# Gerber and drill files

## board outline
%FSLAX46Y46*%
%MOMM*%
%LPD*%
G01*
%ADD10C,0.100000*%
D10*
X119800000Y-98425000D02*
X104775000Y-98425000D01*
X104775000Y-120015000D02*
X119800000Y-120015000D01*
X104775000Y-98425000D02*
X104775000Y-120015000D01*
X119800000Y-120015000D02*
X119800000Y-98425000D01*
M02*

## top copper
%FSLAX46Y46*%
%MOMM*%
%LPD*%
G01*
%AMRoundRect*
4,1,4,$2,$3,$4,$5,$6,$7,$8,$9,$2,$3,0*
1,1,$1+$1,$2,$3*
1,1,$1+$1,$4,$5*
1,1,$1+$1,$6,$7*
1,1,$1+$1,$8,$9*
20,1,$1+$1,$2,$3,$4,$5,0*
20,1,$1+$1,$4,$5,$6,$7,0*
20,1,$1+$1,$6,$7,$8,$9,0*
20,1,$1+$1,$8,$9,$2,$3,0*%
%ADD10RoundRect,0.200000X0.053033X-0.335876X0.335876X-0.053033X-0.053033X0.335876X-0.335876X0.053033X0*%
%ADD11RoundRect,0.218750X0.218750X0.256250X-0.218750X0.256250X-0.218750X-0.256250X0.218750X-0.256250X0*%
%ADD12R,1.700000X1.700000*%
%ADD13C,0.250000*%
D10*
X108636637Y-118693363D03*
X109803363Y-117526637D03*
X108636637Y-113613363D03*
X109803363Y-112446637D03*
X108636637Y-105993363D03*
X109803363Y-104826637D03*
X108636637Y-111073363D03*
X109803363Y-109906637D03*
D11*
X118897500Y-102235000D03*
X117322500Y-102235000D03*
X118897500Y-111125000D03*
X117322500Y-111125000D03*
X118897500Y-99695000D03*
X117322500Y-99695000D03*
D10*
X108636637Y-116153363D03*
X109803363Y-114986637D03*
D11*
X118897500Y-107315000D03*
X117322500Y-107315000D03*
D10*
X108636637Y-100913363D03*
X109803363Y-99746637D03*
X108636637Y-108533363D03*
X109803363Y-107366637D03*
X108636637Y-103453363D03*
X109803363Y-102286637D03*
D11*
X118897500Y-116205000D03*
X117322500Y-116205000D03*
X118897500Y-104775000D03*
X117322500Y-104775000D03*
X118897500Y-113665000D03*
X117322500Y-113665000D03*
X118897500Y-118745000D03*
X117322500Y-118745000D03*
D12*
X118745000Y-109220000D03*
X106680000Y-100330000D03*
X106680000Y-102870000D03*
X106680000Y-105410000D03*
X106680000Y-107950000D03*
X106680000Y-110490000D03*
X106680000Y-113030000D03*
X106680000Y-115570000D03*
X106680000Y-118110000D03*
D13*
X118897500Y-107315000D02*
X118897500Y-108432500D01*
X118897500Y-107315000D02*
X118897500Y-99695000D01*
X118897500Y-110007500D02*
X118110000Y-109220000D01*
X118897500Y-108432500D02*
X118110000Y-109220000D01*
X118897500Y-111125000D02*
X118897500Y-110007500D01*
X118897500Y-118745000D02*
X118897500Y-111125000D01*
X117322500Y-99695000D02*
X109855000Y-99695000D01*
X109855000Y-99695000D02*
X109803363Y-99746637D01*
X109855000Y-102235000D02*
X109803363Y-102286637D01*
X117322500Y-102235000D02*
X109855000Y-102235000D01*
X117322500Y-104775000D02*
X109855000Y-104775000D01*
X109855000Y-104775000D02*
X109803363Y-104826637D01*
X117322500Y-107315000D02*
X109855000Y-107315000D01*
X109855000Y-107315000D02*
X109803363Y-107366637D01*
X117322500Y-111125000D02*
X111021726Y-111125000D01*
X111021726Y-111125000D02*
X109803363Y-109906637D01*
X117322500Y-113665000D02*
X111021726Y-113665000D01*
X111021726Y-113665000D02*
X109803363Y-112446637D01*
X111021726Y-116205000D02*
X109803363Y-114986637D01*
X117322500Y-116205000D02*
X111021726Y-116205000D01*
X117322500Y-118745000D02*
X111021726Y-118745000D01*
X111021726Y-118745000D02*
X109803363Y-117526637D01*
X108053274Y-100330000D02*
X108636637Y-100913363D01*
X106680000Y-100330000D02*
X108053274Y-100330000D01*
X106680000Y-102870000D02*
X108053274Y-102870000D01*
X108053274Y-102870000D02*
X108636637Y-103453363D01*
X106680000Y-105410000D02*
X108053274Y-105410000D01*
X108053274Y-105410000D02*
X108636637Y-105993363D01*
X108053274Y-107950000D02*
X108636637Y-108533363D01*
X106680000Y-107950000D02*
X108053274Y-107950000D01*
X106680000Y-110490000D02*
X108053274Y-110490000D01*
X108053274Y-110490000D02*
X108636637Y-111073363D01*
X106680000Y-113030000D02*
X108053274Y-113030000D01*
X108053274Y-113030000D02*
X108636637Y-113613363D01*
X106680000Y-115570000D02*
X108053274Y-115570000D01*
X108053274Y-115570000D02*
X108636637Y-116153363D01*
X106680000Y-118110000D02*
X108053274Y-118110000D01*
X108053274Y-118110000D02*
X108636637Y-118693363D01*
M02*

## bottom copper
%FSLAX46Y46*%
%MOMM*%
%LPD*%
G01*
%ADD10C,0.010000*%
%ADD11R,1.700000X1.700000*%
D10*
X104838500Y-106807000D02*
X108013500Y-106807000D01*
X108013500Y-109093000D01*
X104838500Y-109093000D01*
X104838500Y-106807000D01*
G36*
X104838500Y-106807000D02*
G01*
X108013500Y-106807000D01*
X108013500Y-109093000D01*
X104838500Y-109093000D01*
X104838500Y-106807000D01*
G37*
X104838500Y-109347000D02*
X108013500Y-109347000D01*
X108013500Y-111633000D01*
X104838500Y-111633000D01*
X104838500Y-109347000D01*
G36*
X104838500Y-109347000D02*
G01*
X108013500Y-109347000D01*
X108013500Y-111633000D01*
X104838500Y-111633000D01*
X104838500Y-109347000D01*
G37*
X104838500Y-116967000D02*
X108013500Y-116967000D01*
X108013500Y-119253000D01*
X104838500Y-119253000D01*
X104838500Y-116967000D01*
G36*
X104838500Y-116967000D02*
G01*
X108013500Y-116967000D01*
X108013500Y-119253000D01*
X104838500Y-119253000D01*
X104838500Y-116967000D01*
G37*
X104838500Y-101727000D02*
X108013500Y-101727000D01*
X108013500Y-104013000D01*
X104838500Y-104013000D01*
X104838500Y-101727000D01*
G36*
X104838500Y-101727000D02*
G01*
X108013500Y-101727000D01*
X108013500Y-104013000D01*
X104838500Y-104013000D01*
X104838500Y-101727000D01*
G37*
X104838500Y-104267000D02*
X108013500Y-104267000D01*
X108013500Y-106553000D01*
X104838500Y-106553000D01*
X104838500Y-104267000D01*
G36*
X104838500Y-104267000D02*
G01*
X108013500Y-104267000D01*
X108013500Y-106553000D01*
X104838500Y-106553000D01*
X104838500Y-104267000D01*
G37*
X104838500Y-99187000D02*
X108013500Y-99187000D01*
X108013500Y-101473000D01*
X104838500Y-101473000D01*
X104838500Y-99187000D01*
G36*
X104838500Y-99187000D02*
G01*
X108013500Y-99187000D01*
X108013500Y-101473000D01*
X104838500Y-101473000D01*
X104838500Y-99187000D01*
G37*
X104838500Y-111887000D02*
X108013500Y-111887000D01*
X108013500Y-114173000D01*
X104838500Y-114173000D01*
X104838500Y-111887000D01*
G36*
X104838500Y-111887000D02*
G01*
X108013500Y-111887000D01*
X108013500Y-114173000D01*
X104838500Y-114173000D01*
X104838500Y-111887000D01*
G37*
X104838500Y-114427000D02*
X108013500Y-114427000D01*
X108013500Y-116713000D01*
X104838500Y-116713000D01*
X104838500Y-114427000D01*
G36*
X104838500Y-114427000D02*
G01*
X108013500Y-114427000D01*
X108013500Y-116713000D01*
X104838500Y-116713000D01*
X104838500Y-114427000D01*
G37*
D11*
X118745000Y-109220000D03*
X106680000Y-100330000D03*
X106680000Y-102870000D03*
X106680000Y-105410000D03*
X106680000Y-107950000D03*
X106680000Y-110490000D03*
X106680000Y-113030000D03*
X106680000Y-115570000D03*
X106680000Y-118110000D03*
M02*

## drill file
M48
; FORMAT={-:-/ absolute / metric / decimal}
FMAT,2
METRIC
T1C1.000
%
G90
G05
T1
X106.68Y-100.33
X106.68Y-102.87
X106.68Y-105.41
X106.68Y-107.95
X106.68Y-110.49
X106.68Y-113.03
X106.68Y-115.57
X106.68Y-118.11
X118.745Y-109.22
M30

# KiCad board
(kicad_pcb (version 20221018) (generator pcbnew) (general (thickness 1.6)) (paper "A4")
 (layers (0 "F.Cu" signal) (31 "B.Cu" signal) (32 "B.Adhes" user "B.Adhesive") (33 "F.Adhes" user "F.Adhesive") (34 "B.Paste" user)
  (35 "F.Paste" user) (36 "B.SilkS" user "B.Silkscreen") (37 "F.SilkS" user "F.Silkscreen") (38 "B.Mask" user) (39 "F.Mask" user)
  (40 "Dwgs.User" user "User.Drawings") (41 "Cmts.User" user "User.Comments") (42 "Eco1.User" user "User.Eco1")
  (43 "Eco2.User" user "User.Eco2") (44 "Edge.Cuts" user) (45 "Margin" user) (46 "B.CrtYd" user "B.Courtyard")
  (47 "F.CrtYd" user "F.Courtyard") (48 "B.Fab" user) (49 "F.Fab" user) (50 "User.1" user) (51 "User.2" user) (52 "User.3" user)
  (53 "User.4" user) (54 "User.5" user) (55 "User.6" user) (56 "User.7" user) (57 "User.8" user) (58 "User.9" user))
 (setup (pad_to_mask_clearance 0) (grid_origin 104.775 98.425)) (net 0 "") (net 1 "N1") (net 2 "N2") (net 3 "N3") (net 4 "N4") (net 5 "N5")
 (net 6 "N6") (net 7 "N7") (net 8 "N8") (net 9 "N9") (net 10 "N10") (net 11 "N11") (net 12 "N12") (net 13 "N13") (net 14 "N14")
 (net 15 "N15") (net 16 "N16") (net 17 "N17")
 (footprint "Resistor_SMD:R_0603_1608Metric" (layer "F.Cu") (at 109.22 118.11 45)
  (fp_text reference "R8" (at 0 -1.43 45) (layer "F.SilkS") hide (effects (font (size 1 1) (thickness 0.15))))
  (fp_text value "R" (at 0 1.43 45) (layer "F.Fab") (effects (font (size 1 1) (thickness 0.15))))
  (pad "1" smd roundrect (at -0.825 0 45) (size 0.8 0.95) (layers "F.Cu" "F.Paste" "F.Mask") (roundrect_rratio 0.25) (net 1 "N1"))
  (pad "2" smd roundrect (at 0.825 0 45) (size 0.8 0.95) (layers "F.Cu" "F.Paste" "F.Mask") (roundrect_rratio 0.25) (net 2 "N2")))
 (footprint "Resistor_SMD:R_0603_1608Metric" (layer "F.Cu") (at 109.22 113.03 45)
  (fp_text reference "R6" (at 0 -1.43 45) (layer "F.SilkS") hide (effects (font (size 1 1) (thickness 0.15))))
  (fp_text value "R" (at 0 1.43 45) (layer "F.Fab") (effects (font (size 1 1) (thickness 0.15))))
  (pad "1" smd roundrect (at -0.825 0 45) (size 0.8 0.95) (layers "F.Cu" "F.Paste" "F.Mask") (roundrect_rratio 0.25) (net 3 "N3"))
  (pad "2" smd roundrect (at 0.825 0 45) (size 0.8 0.95) (layers "F.Cu" "F.Paste" "F.Mask") (roundrect_rratio 0.25) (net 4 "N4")))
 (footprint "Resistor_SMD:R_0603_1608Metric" (layer "F.Cu") (at 109.22 105.41 45)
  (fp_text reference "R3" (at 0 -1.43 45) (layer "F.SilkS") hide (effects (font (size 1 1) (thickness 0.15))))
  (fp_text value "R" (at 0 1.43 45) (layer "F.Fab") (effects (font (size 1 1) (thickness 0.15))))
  (pad "1" smd roundrect (at -0.825 0 45) (size 0.8 0.95) (layers "F.Cu" "F.Paste" "F.Mask") (roundrect_rratio 0.25) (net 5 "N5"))
  (pad "2" smd roundrect (at 0.825 0 45) (size 0.8 0.95) (layers "F.Cu" "F.Paste" "F.Mask") (roundrect_rratio 0.25) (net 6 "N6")))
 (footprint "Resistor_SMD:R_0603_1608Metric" (layer "F.Cu") (at 109.22 110.49 45)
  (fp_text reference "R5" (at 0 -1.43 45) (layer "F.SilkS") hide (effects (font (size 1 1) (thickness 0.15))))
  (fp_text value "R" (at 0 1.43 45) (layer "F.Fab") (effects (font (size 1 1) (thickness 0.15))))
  (pad "1" smd roundrect (at -0.825 0 45) (size 0.8 0.95) (layers "F.Cu" "F.Paste" "F.Mask") (roundrect_rratio 0.25) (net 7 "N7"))
  (pad "2" smd roundrect (at 0.825 0 45) (size 0.8 0.95) (layers "F.Cu" "F.Paste" "F.Mask") (roundrect_rratio 0.25) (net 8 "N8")))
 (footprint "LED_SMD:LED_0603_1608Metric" (layer "F.Cu") (at 118.11 102.235 180)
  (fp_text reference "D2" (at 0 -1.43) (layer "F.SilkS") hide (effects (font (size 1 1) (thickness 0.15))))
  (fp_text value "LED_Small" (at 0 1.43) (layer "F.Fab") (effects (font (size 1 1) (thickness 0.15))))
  (pad "1" smd roundrect (at -0.7875 0 180) (size 0.875 0.95) (layers "F.Cu" "F.Paste" "F.Mask") (roundrect_rratio 0.25) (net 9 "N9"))
  (pad "2" smd roundrect (at 0.7875 0 180) (size 0.875 0.95) (layers "F.Cu" "F.Paste" "F.Mask") (roundrect_rratio 0.25) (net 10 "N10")))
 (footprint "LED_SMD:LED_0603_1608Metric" (layer "F.Cu") (at 118.11 111.125 180)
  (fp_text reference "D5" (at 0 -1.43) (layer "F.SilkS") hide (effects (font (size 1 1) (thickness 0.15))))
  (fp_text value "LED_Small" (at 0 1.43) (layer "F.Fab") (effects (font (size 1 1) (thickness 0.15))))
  (pad "1" smd roundrect (at -0.7875 0 180) (size 0.875 0.95) (layers "F.Cu" "F.Paste" "F.Mask") (roundrect_rratio 0.25) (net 9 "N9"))
  (pad "2" smd roundrect (at 0.7875 0 180) (size 0.875 0.95) (layers "F.Cu" "F.Paste" "F.Mask") (roundrect_rratio 0.25) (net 8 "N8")))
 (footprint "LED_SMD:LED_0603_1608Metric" (layer "F.Cu") (at 118.11 99.695 180)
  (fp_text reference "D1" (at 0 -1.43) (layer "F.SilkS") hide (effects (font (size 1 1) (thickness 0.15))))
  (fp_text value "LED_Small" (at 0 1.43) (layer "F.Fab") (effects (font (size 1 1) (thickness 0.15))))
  (pad "1" smd roundrect (at -0.7875 0 180) (size 0.875 0.95) (layers "F.Cu" "F.Paste" "F.Mask") (roundrect_rratio 0.25) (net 9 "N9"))
  (pad "2" smd roundrect (at 0.7875 0 180) (size 0.875 0.95) (layers "F.Cu" "F.Paste" "F.Mask") (roundrect_rratio 0.25) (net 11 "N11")))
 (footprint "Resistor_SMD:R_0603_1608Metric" (layer "F.Cu") (at 109.22 115.57 45)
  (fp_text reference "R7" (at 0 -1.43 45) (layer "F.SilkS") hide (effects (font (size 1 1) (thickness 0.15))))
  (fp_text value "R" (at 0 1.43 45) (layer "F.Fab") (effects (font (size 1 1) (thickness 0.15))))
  (pad "1" smd roundrect (at -0.825 0 45) (size 0.8 0.95) (layers "F.Cu" "F.Paste" "F.Mask") (roundrect_rratio 0.25) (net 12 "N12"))
  (pad "2" smd roundrect (at 0.825 0 45) (size 0.8 0.95) (layers "F.Cu" "F.Paste" "F.Mask") (roundrect_rratio 0.25) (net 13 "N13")))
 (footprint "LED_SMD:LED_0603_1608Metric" (layer "F.Cu") (at 118.11 107.315 180)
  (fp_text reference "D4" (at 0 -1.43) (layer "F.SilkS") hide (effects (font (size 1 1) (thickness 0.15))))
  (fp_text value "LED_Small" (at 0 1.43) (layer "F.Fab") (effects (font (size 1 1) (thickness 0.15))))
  (pad "1" smd roundrect (at -0.7875 0 180) (size 0.875 0.95) (layers "F.Cu" "F.Paste" "F.Mask") (roundrect_rratio 0.25) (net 9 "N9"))
  (pad "2" smd roundrect (at 0.7875 0 180) (size 0.875 0.95) (layers "F.Cu" "F.Paste" "F.Mask") (roundrect_rratio 0.25) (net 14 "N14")))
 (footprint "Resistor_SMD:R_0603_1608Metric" (layer "F.Cu") (at 109.22 100.33 45)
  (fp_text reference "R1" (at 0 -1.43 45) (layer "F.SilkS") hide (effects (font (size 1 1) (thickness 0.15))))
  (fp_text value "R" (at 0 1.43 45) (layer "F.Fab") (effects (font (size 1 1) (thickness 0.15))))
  (pad "1" smd roundrect (at -0.825 0 45) (size 0.8 0.95) (layers "F.Cu" "F.Paste" "F.Mask") (roundrect_rratio 0.25) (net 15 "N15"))
  (pad "2" smd roundrect (at 0.825 0 45) (size 0.8 0.95) (layers "F.Cu" "F.Paste" "F.Mask") (roundrect_rratio 0.25) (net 11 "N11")))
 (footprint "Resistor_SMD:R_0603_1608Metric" (layer "F.Cu") (at 109.22 107.95 45)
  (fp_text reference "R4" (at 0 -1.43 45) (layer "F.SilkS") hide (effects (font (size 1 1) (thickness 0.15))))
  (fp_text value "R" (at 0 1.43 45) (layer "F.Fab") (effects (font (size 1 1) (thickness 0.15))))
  (pad "1" smd roundrect (at -0.825 0 45) (size 0.8 0.95) (layers "F.Cu" "F.Paste" "F.Mask") (roundrect_rratio 0.25) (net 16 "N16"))
  (pad "2" smd roundrect (at 0.825 0 45) (size 0.8 0.95) (layers "F.Cu" "F.Paste" "F.Mask") (roundrect_rratio 0.25) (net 14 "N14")))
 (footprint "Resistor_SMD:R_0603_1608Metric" (layer "F.Cu") (at 109.22 102.87 45)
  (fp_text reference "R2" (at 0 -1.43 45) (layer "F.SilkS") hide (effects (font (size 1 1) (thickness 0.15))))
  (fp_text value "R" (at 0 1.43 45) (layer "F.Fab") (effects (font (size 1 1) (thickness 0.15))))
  (pad "1" smd roundrect (at -0.825 0 45) (size 0.8 0.95) (layers "F.Cu" "F.Paste" "F.Mask") (roundrect_rratio 0.25) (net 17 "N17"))
  (pad "2" smd roundrect (at 0.825 0 45) (size 0.8 0.95) (layers "F.Cu" "F.Paste" "F.Mask") (roundrect_rratio 0.25) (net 10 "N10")))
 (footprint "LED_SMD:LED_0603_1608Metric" (layer "F.Cu") (at 118.11 116.205 180)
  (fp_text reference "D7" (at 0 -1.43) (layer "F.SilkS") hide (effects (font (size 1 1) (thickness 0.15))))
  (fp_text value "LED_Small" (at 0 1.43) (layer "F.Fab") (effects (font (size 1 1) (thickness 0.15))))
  (pad "1" smd roundrect (at -0.7875 0 180) (size 0.875 0.95) (layers "F.Cu" "F.Paste" "F.Mask") (roundrect_rratio 0.25) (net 9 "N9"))
  (pad "2" smd roundrect (at 0.7875 0 180) (size 0.875 0.95) (layers "F.Cu" "F.Paste" "F.Mask") (roundrect_rratio 0.25) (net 13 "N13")))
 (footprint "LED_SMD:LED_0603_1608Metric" (layer "F.Cu") (at 118.11 104.775 180)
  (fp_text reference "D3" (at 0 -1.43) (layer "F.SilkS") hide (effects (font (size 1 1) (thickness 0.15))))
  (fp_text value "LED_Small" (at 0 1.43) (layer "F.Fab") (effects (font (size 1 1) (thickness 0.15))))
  (pad "1" smd roundrect (at -0.7875 0 180) (size 0.875 0.95) (layers "F.Cu" "F.Paste" "F.Mask") (roundrect_rratio 0.25) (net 9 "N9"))
  (pad "2" smd roundrect (at 0.7875 0 180) (size 0.875 0.95) (layers "F.Cu" "F.Paste" "F.Mask") (roundrect_rratio 0.25) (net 6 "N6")))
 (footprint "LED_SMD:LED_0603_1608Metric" (layer "F.Cu") (at 118.11 113.665 180)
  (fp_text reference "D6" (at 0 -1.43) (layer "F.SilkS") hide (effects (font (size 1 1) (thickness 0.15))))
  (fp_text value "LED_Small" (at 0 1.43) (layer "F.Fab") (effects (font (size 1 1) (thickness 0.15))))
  (pad "1" smd roundrect (at -0.7875 0 180) (size 0.875 0.95) (layers "F.Cu" "F.Paste" "F.Mask") (roundrect_rratio 0.25) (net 9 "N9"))
  (pad "2" smd roundrect (at 0.7875 0 180) (size 0.875 0.95) (layers "F.Cu" "F.Paste" "F.Mask") (roundrect_rratio 0.25) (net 4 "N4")))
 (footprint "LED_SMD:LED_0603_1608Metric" (layer "F.Cu") (at 118.11 118.745 180)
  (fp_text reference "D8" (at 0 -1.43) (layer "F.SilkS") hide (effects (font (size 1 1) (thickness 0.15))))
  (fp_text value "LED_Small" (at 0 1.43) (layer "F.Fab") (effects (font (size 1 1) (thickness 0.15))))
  (pad "1" smd roundrect (at -0.7875 0 180) (size 0.875 0.95) (layers "F.Cu" "F.Paste" "F.Mask") (roundrect_rratio 0.25) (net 9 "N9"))
  (pad "2" smd roundrect (at 0.7875 0 180) (size 0.875 0.95) (layers "F.Cu" "F.Paste" "F.Mask") (roundrect_rratio 0.25) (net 2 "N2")))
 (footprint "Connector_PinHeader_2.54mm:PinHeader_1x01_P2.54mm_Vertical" (layer "F.Cu") (at 118.745 109.22)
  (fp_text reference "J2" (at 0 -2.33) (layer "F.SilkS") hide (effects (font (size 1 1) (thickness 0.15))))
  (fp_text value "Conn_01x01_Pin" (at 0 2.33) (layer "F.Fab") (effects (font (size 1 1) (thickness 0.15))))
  (pad "1" thru_hole rect (at 0 0) (size 1.7 1.7) (drill 1) (layers "*.Cu" "*.Mask") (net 9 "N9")))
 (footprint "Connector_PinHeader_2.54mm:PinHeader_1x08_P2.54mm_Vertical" (layer "B.Cu") (at 106.68 100.33 180)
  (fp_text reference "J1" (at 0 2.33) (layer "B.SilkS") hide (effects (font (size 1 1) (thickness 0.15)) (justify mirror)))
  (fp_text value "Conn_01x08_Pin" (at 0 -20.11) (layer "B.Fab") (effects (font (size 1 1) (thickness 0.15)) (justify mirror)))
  (pad "1" thru_hole rect (at 0 0 180) (size 1.7 1.7) (drill 1) (layers "*.Cu" "*.Mask") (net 15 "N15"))
  (pad "2" thru_hole rect (at 0 -2.54 180) (size 1.7 1.7) (drill 1) (layers "*.Cu" "*.Mask") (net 17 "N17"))
  (pad "3" thru_hole rect (at 0 -5.08 180) (size 1.7 1.7) (drill 1) (layers "*.Cu" "*.Mask") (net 5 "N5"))
  (pad "4" thru_hole rect (at 0 -7.62 180) (size 1.7 1.7) (drill 1) (layers "*.Cu" "*.Mask") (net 16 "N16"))
  (pad "5" thru_hole rect (at 0 -10.16 180) (size 1.7 1.7) (drill 1) (layers "*.Cu" "*.Mask") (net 7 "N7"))
  (pad "6" thru_hole rect (at 0 -12.7 180) (size 1.7 1.7) (drill 1) (layers "*.Cu" "*.Mask") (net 3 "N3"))
  (pad "7" thru_hole rect (at 0 -15.24 180) (size 1.7 1.7) (drill 1) (layers "*.Cu" "*.Mask") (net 12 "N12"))
  (pad "8" thru_hole rect (at 0 -17.78 180) (size 1.7 1.7) (drill 1) (layers "*.Cu" "*.Mask") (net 1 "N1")))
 (gr_rect (start 104.8385 106.807) (end 108.0135 109.093) (stroke (width 0.01) (type solid)) (fill solid) (layer "B.Cu"))
 (gr_rect (start 104.8385 109.347) (end 108.0135 111.633) (stroke (width 0.01) (type solid)) (fill solid) (layer "B.Cu"))
 (gr_rect (start 104.8385 116.967) (end 108.0135 119.253) (stroke (width 0.01) (type solid)) (fill solid) (layer "B.Cu"))
 (gr_rect (start 104.8385 101.727) (end 108.0135 104.013) (stroke (width 0.01) (type solid)) (fill solid) (layer "B.Cu"))
 (gr_rect (start 104.8385 104.267) (end 108.0135 106.553) (stroke (width 0.01) (type solid)) (fill solid) (layer "B.Cu"))
 (gr_rect (start 104.8385 99.187) (end 108.0135 101.473) (stroke (width 0.01) (type solid)) (fill solid) (layer "B.Cu"))
 (gr_rect (start 104.8385 111.887) (end 108.0135 114.173) (stroke (width 0.01) (type solid)) (fill solid) (layer "B.Cu"))
 (gr_rect (start 104.8385 114.427) (end 108.0135 116.713) (stroke (width 0.01) (type solid)) (fill solid) (layer "B.Cu"))
 (gr_line (start 119.8 98.425) (end 104.775 98.425) (stroke (width 0.1) (type default)) (layer "Edge.Cuts"))
 (gr_line (start 104.775 120.015) (end 119.8 120.015) (stroke (width 0.1) (type default)) (layer "Edge.Cuts"))
 (gr_line (start 104.775 98.425) (end 104.775 120.015) (stroke (width 0.1) (type default)) (layer "Edge.Cuts"))
 (gr_line (start 119.8 120.015) (end 119.8 98.425) (stroke (width 0.1) (type default)) (layer "Edge.Cuts"))
 (segment (start 118.8975 107.315) (end 118.8975 108.4325) (width 0.25) (layer "F.Cu") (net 9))
 (segment (start 118.8975 107.315) (end 118.8975 99.695) (width 0.25) (layer "F.Cu") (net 9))
 (segment (start 118.8975 110.0075) (end 118.11 109.22) (width 0.25) (layer "F.Cu") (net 9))
 (segment (start 118.8975 108.4325) (end 118.11 109.22) (width 0.25) (layer "F.Cu") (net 9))
 (segment (start 118.8975 111.125) (end 118.8975 110.0075) (width 0.25) (layer "F.Cu") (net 9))
 (segment (start 118.8975 118.745) (end 118.8975 111.125) (width 0.25) (layer "F.Cu") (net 9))
 (segment (start 117.3225 99.695) (end 109.855 99.695) (width 0.25) (layer "F.Cu") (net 11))
 (segment (start 109.855 99.695) (end 109.803363 99.746637) (width 0.25) (layer "F.Cu") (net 11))
 (segment (start 109.855 102.235) (end 109.803363 102.286637) (width 0.25) (layer "F.Cu") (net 10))
 (segment (start 117.3225 102.235) (end 109.855 102.235) (width 0.25) (layer "F.Cu") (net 10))
 (segment (start 117.3225 104.775) (end 109.855 104.775) (width 0.25) (layer "F.Cu") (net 6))
 (segment (start 109.855 104.775) (end 109.803363 104.826637) (width 0.25) (layer "F.Cu") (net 6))
 (segment (start 117.3225 107.315) (end 109.855 107.315) (width 0.25) (layer "F.Cu") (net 14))
 (segment (start 109.855 107.315) (end 109.803363 107.366637) (width 0.25) (layer "F.Cu") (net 14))
 (segment (start 117.3225 111.125) (end 111.021726 111.125) (width 0.25) (layer "F.Cu") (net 8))
 (segment (start 111.021726 111.125) (end 109.803363 109.906637) (width 0.25) (layer "F.Cu") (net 8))
 (segment (start 117.3225 113.665) (end 111.021726 113.665) (width 0.25) (layer "F.Cu") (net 4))
 (segment (start 111.021726 113.665) (end 109.803363 112.446637) (width 0.25) (layer "F.Cu") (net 4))
 (segment (start 111.021726 116.205) (end 109.803363 114.986637) (width 0.25) (layer "F.Cu") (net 13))
 (segment (start 117.3225 116.205) (end 111.021726 116.205) (width 0.25) (layer "F.Cu") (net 13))
 (segment (start 117.3225 118.745) (end 111.021726 118.745) (width 0.25) (layer "F.Cu") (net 2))
 (segment (start 111.021726 118.745) (end 109.803363 117.526637) (width 0.25) (layer "F.Cu") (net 2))
 (segment (start 108.053274 100.33) (end 108.636637 100.913363) (width 0.25) (layer "F.Cu") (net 15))
 (segment (start 106.68 100.33) (end 108.053274 100.33) (width 0.25) (layer "F.Cu") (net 15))
 (segment (start 106.68 102.87) (end 108.053274 102.87) (width 0.25) (layer "F.Cu") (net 17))
 (segment (start 108.053274 102.87) (end 108.636637 103.453363) (width 0.25) (layer "F.Cu") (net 17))
 (segment (start 106.68 105.41) (end 108.053274 105.41) (width 0.25) (layer "F.Cu") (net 5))
 (segment (start 108.053274 105.41) (end 108.636637 105.993363) (width 0.25) (layer "F.Cu") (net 5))
 (segment (start 108.053274 107.95) (end 108.636637 108.533363) (width 0.25) (layer "F.Cu") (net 16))
 (segment (start 106.68 107.95) (end 108.053274 107.95) (width 0.25) (layer "F.Cu") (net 16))
 (segment (start 106.68 110.49) (end 108.053274 110.49) (width 0.25) (layer "F.Cu") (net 7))
 (segment (start 108.053274 110.49) (end 108.636637 111.073363) (width 0.25) (layer "F.Cu") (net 7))
 (segment (start 106.68 113.03) (end 108.053274 113.03) (width 0.25) (layer "F.Cu") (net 3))
 (segment (start 108.053274 113.03) (end 108.636637 113.613363) (width 0.25) (layer "F.Cu") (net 3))
 (segment (start 106.68 115.57) (end 108.053274 115.57) (width 0.25) (layer "F.Cu") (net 12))
 (segment (start 108.053274 115.57) (end 108.636637 116.153363) (width 0.25) (layer "F.Cu") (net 12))
 (segment (start 106.68 118.11) (end 108.053274 118.11) (width 0.25) (layer "F.Cu") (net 1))
 (segment (start 108.053274 118.11) (end 108.636637 118.693363) (width 0.25) (layer "F.Cu") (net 1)))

